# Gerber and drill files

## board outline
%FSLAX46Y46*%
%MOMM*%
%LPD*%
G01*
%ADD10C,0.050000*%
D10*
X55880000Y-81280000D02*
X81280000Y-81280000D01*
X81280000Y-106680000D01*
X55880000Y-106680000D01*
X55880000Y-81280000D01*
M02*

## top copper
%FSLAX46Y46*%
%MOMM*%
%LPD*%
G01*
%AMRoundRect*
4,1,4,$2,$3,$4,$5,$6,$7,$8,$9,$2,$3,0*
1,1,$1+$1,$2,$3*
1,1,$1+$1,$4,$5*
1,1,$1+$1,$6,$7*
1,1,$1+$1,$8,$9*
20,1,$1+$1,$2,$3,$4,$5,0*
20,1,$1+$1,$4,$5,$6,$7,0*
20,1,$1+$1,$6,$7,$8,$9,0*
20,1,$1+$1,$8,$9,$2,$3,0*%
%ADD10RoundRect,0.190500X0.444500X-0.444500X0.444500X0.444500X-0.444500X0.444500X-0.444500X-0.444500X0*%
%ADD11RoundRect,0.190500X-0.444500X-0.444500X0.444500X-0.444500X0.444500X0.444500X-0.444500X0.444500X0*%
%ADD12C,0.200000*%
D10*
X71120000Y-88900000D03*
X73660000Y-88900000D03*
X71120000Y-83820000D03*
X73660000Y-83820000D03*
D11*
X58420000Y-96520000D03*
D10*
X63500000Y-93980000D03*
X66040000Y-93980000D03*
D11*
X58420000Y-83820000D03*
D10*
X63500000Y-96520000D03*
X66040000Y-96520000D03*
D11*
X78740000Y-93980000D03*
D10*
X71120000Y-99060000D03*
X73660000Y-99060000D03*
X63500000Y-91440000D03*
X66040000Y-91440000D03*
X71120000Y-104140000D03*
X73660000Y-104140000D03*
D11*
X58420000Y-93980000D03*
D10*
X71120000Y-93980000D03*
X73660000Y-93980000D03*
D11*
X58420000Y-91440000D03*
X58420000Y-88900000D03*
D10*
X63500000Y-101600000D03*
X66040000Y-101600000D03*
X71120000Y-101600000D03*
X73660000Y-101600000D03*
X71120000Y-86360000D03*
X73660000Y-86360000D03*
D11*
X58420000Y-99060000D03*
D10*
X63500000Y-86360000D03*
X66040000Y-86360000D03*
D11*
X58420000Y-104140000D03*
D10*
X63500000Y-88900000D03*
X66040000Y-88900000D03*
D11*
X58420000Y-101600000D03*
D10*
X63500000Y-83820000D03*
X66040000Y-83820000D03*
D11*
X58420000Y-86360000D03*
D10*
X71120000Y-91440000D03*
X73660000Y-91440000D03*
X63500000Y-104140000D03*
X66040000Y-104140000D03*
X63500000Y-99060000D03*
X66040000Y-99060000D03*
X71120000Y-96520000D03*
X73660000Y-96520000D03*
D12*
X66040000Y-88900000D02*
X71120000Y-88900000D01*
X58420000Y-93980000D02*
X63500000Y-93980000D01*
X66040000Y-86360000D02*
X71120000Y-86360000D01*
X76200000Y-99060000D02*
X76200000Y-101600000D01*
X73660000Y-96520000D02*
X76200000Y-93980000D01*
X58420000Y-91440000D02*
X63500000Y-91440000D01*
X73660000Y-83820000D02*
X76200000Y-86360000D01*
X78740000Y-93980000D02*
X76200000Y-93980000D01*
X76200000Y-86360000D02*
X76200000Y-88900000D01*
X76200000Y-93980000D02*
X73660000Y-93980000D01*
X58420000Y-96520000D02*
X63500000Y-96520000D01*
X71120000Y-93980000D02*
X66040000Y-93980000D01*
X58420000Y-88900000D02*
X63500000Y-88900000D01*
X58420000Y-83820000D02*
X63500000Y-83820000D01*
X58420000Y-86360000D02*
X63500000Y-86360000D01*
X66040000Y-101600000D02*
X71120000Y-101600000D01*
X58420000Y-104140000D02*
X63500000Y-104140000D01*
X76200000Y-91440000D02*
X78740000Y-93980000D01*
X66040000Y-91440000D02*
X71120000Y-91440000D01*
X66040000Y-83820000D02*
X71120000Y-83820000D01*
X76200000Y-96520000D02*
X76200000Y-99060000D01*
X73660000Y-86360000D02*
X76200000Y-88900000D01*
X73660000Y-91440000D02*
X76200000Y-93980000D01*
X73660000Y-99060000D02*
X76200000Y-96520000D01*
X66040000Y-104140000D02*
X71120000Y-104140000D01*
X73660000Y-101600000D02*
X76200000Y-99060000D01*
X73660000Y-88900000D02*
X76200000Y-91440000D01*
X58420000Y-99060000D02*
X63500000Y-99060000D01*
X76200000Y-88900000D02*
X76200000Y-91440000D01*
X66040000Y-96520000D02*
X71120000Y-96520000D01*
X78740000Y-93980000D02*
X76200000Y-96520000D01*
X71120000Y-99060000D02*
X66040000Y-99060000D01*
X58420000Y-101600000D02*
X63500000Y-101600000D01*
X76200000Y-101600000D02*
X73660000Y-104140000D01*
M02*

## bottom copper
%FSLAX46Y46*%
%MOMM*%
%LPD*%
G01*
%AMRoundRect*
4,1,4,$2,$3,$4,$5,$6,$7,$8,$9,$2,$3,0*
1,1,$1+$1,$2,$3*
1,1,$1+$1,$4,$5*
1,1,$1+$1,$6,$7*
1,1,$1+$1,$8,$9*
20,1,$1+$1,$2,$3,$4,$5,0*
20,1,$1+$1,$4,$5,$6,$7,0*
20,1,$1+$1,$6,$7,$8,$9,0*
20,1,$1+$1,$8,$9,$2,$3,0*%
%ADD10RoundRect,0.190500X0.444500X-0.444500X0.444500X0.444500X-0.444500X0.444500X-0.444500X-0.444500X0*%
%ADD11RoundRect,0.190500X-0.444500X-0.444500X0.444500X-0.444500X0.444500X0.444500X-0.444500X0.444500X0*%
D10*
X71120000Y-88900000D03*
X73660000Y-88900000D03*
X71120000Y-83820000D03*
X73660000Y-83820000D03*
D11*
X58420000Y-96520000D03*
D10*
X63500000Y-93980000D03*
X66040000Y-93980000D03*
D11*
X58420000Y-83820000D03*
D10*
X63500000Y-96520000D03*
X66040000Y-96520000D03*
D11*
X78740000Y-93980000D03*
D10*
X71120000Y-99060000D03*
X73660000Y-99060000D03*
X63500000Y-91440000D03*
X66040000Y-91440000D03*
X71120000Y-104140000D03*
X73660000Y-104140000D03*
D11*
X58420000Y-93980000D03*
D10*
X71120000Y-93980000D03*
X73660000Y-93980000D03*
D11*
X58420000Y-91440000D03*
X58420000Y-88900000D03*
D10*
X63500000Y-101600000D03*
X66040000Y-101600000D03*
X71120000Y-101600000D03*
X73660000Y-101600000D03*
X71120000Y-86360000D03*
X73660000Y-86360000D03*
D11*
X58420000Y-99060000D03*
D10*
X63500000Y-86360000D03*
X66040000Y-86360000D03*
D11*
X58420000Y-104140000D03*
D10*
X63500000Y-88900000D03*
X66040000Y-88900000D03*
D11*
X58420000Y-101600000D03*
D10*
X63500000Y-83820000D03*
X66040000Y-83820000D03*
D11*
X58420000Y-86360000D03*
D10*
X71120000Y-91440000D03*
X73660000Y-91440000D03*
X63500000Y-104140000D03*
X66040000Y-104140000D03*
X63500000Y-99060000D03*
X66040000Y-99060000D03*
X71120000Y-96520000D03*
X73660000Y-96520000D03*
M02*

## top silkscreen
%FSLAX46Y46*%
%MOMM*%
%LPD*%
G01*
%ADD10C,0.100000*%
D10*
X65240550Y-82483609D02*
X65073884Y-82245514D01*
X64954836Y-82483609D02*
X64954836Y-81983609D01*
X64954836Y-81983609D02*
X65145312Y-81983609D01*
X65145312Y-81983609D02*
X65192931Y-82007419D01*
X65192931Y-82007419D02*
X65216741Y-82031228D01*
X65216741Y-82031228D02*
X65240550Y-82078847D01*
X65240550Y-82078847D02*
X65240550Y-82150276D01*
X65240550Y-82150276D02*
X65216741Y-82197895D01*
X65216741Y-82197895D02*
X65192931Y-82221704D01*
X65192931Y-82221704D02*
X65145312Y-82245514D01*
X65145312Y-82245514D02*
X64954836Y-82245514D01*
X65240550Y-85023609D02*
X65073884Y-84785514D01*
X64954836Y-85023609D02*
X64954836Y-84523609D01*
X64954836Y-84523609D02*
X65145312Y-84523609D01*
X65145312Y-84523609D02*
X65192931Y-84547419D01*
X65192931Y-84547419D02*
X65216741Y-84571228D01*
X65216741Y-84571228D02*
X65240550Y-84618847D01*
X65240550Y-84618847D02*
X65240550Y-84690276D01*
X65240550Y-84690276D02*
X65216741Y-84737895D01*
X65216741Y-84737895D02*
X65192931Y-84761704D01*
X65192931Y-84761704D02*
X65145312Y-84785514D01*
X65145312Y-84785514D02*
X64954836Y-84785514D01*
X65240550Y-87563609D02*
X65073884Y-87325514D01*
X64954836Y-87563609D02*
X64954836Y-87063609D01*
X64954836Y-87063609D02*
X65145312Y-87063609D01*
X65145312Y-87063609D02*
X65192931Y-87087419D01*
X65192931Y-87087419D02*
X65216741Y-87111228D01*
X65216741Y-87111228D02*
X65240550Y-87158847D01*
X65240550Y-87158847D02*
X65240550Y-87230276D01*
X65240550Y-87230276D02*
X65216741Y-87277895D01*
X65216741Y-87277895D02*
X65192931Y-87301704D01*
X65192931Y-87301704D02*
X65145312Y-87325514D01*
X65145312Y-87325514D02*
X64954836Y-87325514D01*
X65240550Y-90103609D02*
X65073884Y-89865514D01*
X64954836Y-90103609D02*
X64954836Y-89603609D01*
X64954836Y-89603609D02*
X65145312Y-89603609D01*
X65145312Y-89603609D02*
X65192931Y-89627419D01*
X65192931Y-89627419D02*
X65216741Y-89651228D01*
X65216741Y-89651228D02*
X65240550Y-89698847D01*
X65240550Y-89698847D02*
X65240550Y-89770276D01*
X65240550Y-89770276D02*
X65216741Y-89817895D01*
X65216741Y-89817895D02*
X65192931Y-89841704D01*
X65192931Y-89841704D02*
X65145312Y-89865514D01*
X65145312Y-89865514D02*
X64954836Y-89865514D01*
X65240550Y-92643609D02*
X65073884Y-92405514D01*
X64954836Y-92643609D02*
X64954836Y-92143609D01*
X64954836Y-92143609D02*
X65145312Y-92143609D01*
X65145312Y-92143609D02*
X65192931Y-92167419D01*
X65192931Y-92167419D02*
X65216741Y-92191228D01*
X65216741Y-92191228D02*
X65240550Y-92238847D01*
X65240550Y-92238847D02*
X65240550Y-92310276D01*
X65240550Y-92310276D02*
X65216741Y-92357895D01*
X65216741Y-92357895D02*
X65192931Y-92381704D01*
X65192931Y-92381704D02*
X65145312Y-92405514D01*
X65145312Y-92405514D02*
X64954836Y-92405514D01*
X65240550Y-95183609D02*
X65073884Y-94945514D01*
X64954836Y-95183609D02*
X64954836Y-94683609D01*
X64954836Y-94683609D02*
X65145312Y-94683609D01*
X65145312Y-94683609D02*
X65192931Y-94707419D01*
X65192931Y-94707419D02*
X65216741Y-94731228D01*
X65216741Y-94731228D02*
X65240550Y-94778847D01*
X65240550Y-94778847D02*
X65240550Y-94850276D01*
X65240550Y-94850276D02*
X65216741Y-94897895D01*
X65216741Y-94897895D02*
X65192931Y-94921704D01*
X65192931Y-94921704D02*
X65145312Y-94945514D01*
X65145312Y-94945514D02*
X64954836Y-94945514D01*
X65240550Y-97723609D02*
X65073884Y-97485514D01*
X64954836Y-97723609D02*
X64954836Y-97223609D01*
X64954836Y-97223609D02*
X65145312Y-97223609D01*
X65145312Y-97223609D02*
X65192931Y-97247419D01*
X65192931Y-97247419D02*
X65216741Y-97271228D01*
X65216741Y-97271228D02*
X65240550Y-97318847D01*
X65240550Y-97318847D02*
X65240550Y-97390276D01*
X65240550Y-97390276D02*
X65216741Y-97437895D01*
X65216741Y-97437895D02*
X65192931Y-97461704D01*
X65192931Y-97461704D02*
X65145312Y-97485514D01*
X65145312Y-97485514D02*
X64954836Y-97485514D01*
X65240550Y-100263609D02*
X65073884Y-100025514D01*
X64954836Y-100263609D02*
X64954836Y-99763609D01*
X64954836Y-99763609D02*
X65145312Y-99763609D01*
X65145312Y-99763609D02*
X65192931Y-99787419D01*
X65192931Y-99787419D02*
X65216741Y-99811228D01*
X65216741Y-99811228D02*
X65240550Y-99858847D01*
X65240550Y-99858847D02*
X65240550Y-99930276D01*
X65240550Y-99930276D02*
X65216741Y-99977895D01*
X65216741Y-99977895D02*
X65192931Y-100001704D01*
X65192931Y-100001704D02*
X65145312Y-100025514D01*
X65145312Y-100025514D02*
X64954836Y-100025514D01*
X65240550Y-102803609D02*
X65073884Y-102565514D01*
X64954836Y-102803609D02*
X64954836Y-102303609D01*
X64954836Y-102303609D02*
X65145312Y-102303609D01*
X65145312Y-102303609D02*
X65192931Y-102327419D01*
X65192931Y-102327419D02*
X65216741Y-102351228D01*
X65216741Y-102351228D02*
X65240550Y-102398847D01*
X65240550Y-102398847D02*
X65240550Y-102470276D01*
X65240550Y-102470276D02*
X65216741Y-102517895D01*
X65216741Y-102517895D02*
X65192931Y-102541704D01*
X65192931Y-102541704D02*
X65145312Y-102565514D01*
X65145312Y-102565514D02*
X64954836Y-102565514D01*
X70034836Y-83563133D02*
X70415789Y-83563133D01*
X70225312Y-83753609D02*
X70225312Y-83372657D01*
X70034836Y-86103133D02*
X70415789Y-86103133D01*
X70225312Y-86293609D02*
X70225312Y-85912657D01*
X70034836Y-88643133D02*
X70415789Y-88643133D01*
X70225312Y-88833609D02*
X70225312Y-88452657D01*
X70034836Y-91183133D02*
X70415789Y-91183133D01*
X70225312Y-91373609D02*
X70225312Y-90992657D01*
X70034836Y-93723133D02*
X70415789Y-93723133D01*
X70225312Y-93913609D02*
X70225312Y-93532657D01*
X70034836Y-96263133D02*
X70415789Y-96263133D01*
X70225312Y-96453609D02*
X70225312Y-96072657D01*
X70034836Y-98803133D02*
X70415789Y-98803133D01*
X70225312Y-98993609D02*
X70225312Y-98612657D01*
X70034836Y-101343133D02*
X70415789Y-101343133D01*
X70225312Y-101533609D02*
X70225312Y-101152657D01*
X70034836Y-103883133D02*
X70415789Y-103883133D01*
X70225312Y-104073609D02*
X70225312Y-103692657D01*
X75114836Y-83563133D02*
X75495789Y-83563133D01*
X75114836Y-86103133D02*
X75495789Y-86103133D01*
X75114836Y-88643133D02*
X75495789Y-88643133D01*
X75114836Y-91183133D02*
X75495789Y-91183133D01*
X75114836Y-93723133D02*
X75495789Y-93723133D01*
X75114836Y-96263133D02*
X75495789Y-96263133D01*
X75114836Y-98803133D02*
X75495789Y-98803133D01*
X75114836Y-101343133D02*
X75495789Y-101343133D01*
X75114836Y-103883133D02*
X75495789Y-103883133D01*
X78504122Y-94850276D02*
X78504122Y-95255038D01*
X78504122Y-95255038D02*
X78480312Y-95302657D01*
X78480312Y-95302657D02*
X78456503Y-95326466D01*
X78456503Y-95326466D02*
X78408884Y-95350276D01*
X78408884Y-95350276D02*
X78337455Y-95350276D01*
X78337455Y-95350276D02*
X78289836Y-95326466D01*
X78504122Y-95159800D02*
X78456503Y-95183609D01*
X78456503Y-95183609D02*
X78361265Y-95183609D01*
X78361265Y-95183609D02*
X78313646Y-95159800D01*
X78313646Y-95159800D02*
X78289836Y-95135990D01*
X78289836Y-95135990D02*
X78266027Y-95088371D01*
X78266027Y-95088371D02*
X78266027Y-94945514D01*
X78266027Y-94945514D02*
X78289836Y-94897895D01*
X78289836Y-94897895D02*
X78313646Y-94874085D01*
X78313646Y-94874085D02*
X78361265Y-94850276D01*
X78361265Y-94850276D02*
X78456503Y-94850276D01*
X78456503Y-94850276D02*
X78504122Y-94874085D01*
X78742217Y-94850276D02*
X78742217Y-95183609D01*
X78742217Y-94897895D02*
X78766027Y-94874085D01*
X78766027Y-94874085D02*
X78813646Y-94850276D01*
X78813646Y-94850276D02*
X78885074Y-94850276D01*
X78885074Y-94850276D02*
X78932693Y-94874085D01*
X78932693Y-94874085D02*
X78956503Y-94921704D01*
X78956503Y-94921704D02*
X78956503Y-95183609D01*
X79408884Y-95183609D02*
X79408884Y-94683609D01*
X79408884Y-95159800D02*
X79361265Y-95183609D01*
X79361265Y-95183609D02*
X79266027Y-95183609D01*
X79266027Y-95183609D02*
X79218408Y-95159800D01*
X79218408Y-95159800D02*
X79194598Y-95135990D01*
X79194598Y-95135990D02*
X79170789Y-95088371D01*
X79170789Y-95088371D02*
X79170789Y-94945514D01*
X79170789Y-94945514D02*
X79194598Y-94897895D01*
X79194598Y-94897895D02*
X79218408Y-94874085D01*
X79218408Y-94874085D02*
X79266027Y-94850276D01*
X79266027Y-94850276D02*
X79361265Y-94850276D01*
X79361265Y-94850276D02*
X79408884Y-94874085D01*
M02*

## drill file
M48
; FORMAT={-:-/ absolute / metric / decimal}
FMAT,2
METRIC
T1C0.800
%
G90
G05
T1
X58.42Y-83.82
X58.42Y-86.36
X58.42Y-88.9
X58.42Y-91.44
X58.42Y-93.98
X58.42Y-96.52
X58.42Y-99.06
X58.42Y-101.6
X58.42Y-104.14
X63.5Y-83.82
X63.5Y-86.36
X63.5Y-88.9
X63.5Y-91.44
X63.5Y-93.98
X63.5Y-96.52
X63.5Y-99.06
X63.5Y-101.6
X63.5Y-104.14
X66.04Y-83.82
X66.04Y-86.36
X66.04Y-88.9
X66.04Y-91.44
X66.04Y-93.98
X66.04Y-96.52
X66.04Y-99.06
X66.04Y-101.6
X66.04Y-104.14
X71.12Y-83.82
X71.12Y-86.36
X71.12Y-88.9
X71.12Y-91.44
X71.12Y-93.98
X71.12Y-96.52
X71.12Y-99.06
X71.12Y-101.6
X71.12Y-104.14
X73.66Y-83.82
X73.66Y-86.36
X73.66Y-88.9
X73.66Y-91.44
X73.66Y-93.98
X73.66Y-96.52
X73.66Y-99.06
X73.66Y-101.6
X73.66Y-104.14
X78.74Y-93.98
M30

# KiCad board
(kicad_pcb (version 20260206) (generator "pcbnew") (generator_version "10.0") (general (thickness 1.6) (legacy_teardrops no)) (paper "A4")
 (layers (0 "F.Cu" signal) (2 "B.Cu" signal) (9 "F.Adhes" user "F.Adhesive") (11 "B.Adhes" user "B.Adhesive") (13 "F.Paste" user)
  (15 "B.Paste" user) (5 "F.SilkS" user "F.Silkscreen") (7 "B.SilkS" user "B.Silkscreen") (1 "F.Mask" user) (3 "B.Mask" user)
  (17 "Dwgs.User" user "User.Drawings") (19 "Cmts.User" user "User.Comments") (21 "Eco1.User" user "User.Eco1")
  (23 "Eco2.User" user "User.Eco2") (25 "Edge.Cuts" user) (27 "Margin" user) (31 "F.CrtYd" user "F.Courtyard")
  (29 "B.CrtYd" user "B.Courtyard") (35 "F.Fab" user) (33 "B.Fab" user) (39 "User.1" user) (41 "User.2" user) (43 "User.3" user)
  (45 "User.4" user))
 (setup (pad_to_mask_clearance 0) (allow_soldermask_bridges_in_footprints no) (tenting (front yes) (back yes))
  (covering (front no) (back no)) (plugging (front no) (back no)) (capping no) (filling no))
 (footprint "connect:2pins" (layer "F.Cu") (at 68.58 88.9 90)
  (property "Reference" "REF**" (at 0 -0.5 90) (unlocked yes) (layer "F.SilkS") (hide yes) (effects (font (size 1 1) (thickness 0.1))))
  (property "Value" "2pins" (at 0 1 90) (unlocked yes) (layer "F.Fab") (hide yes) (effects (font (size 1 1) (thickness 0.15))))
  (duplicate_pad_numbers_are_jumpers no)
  (pad "1" thru_hole roundrect (at 0 2.54 90) (size 1.27 1.27) (drill 0.8) (layers "*.Cu" "*.Mask") (remove_unused_layers no)
   (roundrect_rratio 0.15))
  (pad "2" thru_hole roundrect (at 0 5.08 90) (size 1.27 1.27) (drill 0.8) (layers "*.Cu" "*.Mask") (remove_unused_layers no)
   (roundrect_rratio 0.15)))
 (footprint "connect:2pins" (layer "F.Cu") (at 68.58 83.82 90)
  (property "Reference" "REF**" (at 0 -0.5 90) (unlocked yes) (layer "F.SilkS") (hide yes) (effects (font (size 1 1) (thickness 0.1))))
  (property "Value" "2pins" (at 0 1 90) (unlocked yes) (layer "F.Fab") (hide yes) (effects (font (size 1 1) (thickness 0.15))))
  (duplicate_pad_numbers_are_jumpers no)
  (pad "1" thru_hole roundrect (at 0 2.54 90) (size 1.27 1.27) (drill 0.8) (layers "*.Cu" "*.Mask") (remove_unused_layers no)
   (roundrect_rratio 0.15))
  (pad "2" thru_hole roundrect (at 0 5.08 90) (size 1.27 1.27) (drill 0.8) (layers "*.Cu" "*.Mask") (remove_unused_layers no)
   (roundrect_rratio 0.15)))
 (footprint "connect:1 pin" (layer "F.Cu") (at 58.42 93.98)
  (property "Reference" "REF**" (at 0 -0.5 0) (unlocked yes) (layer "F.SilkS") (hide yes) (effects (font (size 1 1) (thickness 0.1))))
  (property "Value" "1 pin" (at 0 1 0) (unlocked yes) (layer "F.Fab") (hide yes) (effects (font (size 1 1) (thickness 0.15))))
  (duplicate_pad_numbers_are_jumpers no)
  (pad "1" thru_hole roundrect (at 0 2.54) (size 1.27 1.27) (drill 0.8) (layers "*.Cu" "*.Mask") (remove_unused_layers no)
   (roundrect_rratio 0.15)))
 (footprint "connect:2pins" (layer "F.Cu") (at 60.96 93.98 90)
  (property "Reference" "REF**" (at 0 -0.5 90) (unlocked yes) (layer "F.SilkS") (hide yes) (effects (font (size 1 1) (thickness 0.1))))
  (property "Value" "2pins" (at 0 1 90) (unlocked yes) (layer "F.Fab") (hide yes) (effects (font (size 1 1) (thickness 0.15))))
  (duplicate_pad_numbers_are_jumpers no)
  (pad "1" thru_hole roundrect (at 0 2.54 90) (size 1.27 1.27) (drill 0.8) (layers "*.Cu" "*.Mask") (remove_unused_layers no)
   (roundrect_rratio 0.15))
  (pad "2" thru_hole roundrect (at 0 5.08 90) (size 1.27 1.27) (drill 0.8) (layers "*.Cu" "*.Mask") (remove_unused_layers no)
   (roundrect_rratio 0.15)))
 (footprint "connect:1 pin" (layer "F.Cu") (at 58.42 81.28)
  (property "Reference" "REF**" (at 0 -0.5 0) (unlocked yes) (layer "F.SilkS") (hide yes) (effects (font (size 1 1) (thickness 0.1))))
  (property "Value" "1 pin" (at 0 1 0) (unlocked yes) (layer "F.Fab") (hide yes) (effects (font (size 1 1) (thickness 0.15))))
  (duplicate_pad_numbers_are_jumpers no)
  (pad "1" thru_hole roundrect (at 0 2.54) (size 1.27 1.27) (drill 0.8) (layers "*.Cu" "*.Mask") (remove_unused_layers no)
   (roundrect_rratio 0.15)))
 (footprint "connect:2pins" (layer "F.Cu") (at 60.96 96.52 90)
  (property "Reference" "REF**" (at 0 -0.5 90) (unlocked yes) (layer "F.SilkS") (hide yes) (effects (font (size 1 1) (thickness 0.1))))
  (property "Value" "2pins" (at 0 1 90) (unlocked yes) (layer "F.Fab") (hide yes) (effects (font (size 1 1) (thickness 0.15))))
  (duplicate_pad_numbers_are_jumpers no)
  (pad "1" thru_hole roundrect (at 0 2.54 90) (size 1.27 1.27) (drill 0.8) (layers "*.Cu" "*.Mask") (remove_unused_layers no)
   (roundrect_rratio 0.15))
  (pad "2" thru_hole roundrect (at 0 5.08 90) (size 1.27 1.27) (drill 0.8) (layers "*.Cu" "*.Mask") (remove_unused_layers no)
   (roundrect_rratio 0.15)))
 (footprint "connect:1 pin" (layer "F.Cu") (at 78.74 91.44)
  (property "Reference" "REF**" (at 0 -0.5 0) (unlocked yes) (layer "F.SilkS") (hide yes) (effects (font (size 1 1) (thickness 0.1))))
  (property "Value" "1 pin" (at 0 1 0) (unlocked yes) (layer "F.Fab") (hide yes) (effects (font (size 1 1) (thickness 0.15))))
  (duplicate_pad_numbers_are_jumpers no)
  (pad "1" thru_hole roundrect (at 0 2.54) (size 1.27 1.27) (drill 0.8) (layers "*.Cu" "*.Mask") (remove_unused_layers no)
   (roundrect_rratio 0.15)))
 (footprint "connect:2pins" (layer "F.Cu") (at 68.58 99.06 90)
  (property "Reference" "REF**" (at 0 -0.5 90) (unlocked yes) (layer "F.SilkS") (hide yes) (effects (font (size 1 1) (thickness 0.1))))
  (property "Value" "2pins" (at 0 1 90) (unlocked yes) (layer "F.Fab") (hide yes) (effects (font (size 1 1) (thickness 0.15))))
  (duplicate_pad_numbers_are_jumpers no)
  (pad "1" thru_hole roundrect (at 0 2.54 90) (size 1.27 1.27) (drill 0.8) (layers "*.Cu" "*.Mask") (remove_unused_layers no)
   (roundrect_rratio 0.15))
  (pad "2" thru_hole roundrect (at 0 5.08 90) (size 1.27 1.27) (drill 0.8) (layers "*.Cu" "*.Mask") (remove_unused_layers no)
   (roundrect_rratio 0.15)))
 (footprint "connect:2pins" (layer "F.Cu") (at 60.96 91.44 90)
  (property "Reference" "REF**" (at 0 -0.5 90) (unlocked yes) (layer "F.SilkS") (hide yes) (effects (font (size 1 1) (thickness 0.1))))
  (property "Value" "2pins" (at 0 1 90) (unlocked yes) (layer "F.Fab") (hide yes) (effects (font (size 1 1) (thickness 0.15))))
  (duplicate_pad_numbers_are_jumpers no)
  (pad "1" thru_hole roundrect (at 0 2.54 90) (size 1.27 1.27) (drill 0.8) (layers "*.Cu" "*.Mask") (remove_unused_layers no)
   (roundrect_rratio 0.15))
  (pad "2" thru_hole roundrect (at 0 5.08 90) (size 1.27 1.27) (drill 0.8) (layers "*.Cu" "*.Mask") (remove_unused_layers no)
   (roundrect_rratio 0.15)))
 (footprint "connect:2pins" (layer "F.Cu") (at 68.58 104.14 90)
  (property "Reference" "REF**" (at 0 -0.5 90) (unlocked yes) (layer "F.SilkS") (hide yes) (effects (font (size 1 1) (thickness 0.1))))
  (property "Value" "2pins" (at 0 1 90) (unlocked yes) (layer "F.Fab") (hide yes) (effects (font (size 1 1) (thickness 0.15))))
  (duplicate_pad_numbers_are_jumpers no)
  (pad "1" thru_hole roundrect (at 0 2.54 90) (size 1.27 1.27) (drill 0.8) (layers "*.Cu" "*.Mask") (remove_unused_layers no)
   (roundrect_rratio 0.15))
  (pad "2" thru_hole roundrect (at 0 5.08 90) (size 1.27 1.27) (drill 0.8) (layers "*.Cu" "*.Mask") (remove_unused_layers no)
   (roundrect_rratio 0.15)))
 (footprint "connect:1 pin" (layer "F.Cu") (at 58.42 91.44)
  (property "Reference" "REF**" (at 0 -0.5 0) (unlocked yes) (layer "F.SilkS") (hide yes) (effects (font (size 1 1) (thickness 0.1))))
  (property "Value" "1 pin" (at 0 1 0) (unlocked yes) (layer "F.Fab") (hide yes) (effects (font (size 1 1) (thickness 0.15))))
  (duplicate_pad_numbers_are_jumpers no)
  (pad "1" thru_hole roundrect (at 0 2.54) (size 1.27 1.27) (drill 0.8) (layers "*.Cu" "*.Mask") (remove_unused_layers no)
   (roundrect_rratio 0.15)))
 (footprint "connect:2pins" (layer "F.Cu") (at 68.58 93.98 90)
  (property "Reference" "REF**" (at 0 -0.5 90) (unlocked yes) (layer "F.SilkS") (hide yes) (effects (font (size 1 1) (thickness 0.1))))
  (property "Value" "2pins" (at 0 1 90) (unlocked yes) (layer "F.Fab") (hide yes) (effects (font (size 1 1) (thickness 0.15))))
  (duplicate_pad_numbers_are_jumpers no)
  (pad "1" thru_hole roundrect (at 0 2.54 90) (size 1.27 1.27) (drill 0.8) (layers "*.Cu" "*.Mask") (remove_unused_layers no)
   (roundrect_rratio 0.15))
  (pad "2" thru_hole roundrect (at 0 5.08 90) (size 1.27 1.27) (drill 0.8) (layers "*.Cu" "*.Mask") (remove_unused_layers no)
   (roundrect_rratio 0.15)))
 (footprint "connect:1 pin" (layer "F.Cu") (at 58.42 88.9)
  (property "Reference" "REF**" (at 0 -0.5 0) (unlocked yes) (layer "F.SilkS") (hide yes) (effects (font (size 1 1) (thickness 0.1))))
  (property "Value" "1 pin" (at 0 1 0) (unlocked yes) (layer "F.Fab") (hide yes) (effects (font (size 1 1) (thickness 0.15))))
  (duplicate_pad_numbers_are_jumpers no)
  (pad "1" thru_hole roundrect (at 0 2.54) (size 1.27 1.27) (drill 0.8) (layers "*.Cu" "*.Mask") (remove_unused_layers no)
   (roundrect_rratio 0.15)))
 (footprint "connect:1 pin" (layer "F.Cu") (at 58.42 86.36)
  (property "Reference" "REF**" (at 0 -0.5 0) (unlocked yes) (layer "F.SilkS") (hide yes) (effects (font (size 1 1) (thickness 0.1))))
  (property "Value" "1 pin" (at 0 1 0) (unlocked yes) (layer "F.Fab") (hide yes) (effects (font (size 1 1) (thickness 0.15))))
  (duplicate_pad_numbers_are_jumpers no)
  (pad "1" thru_hole roundrect (at 0 2.54) (size 1.27 1.27) (drill 0.8) (layers "*.Cu" "*.Mask") (remove_unused_layers no)
   (roundrect_rratio 0.15)))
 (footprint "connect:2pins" (layer "F.Cu") (at 60.96 101.6 90)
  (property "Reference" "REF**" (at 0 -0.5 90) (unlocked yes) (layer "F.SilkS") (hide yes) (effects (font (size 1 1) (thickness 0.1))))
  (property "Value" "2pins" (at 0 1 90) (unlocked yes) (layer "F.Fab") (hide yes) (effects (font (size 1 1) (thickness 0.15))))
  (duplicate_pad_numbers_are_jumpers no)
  (pad "1" thru_hole roundrect (at 0 2.54 90) (size 1.27 1.27) (drill 0.8) (layers "*.Cu" "*.Mask") (remove_unused_layers no)
   (roundrect_rratio 0.15))
  (pad "2" thru_hole roundrect (at 0 5.08 90) (size 1.27 1.27) (drill 0.8) (layers "*.Cu" "*.Mask") (remove_unused_layers no)
   (roundrect_rratio 0.15)))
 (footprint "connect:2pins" (layer "F.Cu") (at 68.58 101.6 90)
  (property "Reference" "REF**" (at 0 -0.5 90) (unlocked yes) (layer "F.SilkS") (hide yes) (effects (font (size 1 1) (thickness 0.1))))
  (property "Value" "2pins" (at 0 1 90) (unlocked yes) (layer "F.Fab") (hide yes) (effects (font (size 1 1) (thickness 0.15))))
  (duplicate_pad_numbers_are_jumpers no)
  (pad "1" thru_hole roundrect (at 0 2.54 90) (size 1.27 1.27) (drill 0.8) (layers "*.Cu" "*.Mask") (remove_unused_layers no)
   (roundrect_rratio 0.15))
  (pad "2" thru_hole roundrect (at 0 5.08 90) (size 1.27 1.27) (drill 0.8) (layers "*.Cu" "*.Mask") (remove_unused_layers no)
   (roundrect_rratio 0.15)))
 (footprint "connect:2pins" (layer "F.Cu") (at 68.58 86.36 90)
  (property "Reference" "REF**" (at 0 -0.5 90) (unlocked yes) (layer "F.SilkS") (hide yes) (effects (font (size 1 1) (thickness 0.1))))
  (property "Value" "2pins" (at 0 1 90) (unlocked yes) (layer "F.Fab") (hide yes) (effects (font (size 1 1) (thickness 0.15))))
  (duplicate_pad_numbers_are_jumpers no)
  (pad "1" thru_hole roundrect (at 0 2.54 90) (size 1.27 1.27) (drill 0.8) (layers "*.Cu" "*.Mask") (remove_unused_layers no)
   (roundrect_rratio 0.15))
  (pad "2" thru_hole roundrect (at 0 5.08 90) (size 1.27 1.27) (drill 0.8) (layers "*.Cu" "*.Mask") (remove_unused_layers no)
   (roundrect_rratio 0.15)))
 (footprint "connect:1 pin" (layer "F.Cu") (at 58.42 96.52)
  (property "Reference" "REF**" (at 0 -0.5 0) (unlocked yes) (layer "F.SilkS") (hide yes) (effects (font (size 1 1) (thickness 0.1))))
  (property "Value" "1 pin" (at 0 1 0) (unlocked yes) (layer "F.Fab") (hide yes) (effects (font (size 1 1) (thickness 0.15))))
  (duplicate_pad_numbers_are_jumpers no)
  (pad "1" thru_hole roundrect (at 0 2.54) (size 1.27 1.27) (drill 0.8) (layers "*.Cu" "*.Mask") (remove_unused_layers no)
   (roundrect_rratio 0.15)))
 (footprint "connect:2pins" (layer "F.Cu") (at 60.96 86.36 90)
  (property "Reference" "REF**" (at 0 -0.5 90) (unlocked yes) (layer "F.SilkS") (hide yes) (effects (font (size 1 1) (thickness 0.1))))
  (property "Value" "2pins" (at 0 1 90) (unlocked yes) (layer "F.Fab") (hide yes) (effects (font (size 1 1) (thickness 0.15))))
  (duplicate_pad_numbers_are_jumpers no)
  (pad "1" thru_hole roundrect (at 0 2.54 90) (size 1.27 1.27) (drill 0.8) (layers "*.Cu" "*.Mask") (remove_unused_layers no)
   (roundrect_rratio 0.15))
  (pad "2" thru_hole roundrect (at 0 5.08 90) (size 1.27 1.27) (drill 0.8) (layers "*.Cu" "*.Mask") (remove_unused_layers no)
   (roundrect_rratio 0.15)))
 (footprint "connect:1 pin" (layer "F.Cu") (at 58.42 101.6)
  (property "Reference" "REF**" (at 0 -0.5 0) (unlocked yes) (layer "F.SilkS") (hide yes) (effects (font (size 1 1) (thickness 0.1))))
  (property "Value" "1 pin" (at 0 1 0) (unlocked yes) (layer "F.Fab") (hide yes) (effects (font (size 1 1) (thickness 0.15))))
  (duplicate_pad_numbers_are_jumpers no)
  (pad "1" thru_hole roundrect (at 0 2.54) (size 1.27 1.27) (drill 0.8) (layers "*.Cu" "*.Mask") (remove_unused_layers no)
   (roundrect_rratio 0.15)))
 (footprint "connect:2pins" (layer "F.Cu") (at 60.96 88.9 90)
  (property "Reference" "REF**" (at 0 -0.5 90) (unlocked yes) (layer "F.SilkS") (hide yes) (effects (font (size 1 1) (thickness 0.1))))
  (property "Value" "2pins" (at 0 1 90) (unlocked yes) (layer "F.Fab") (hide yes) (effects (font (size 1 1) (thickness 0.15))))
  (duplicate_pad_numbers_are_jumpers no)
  (pad "1" thru_hole roundrect (at 0 2.54 90) (size 1.27 1.27) (drill 0.8) (layers "*.Cu" "*.Mask") (remove_unused_layers no)
   (roundrect_rratio 0.15))
  (pad "2" thru_hole roundrect (at 0 5.08 90) (size 1.27 1.27) (drill 0.8) (layers "*.Cu" "*.Mask") (remove_unused_layers no)
   (roundrect_rratio 0.15)))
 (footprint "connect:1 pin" (layer "F.Cu") (at 58.42 99.06)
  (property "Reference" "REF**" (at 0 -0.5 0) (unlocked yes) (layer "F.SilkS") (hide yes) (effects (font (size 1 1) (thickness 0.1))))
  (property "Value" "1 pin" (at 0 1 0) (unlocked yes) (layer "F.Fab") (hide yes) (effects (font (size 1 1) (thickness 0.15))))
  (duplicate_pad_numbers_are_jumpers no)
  (pad "1" thru_hole roundrect (at 0 2.54) (size 1.27 1.27) (drill 0.8) (layers "*.Cu" "*.Mask") (remove_unused_layers no)
   (roundrect_rratio 0.15)))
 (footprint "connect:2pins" (layer "F.Cu") (at 60.96 83.82 90)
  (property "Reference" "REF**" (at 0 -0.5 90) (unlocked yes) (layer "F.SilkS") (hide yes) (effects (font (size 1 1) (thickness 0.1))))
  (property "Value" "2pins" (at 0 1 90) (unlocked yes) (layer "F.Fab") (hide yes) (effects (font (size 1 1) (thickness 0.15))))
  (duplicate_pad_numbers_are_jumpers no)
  (pad "1" thru_hole roundrect (at 0 2.54 90) (size 1.27 1.27) (drill 0.8) (layers "*.Cu" "*.Mask") (remove_unused_layers no)
   (roundrect_rratio 0.15))
  (pad "2" thru_hole roundrect (at 0 5.08 90) (size 1.27 1.27) (drill 0.8) (layers "*.Cu" "*.Mask") (remove_unused_layers no)
   (roundrect_rratio 0.15)))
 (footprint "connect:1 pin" (layer "F.Cu") (at 58.42 83.82)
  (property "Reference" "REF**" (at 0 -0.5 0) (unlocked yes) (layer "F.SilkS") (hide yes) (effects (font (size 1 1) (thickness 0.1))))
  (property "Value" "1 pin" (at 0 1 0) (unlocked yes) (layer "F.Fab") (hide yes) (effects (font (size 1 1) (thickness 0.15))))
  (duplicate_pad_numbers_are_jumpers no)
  (pad "1" thru_hole roundrect (at 0 2.54) (size 1.27 1.27) (drill 0.8) (layers "*.Cu" "*.Mask") (remove_unused_layers no)
   (roundrect_rratio 0.15)))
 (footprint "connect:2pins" (layer "F.Cu") (at 68.58 91.44 90)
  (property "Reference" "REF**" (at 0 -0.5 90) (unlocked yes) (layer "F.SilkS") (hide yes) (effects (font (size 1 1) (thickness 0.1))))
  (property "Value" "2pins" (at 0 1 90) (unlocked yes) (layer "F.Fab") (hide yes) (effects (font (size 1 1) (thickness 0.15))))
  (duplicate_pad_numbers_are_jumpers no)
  (pad "1" thru_hole roundrect (at 0 2.54 90) (size 1.27 1.27) (drill 0.8) (layers "*.Cu" "*.Mask") (remove_unused_layers no)
   (roundrect_rratio 0.15))
  (pad "2" thru_hole roundrect (at 0 5.08 90) (size 1.27 1.27) (drill 0.8) (layers "*.Cu" "*.Mask") (remove_unused_layers no)
   (roundrect_rratio 0.15)))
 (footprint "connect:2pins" (layer "F.Cu") (at 60.96 104.14 90)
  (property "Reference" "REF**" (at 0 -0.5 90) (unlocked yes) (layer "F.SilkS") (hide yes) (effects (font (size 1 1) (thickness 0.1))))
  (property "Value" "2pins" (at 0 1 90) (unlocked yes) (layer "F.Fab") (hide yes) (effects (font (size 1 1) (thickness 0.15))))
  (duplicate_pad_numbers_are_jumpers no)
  (pad "1" thru_hole roundrect (at 0 2.54 90) (size 1.27 1.27) (drill 0.8) (layers "*.Cu" "*.Mask") (remove_unused_layers no)
   (roundrect_rratio 0.15))
  (pad "2" thru_hole roundrect (at 0 5.08 90) (size 1.27 1.27) (drill 0.8) (layers "*.Cu" "*.Mask") (remove_unused_layers no)
   (roundrect_rratio 0.15)))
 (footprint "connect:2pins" (layer "F.Cu") (at 60.96 99.06 90)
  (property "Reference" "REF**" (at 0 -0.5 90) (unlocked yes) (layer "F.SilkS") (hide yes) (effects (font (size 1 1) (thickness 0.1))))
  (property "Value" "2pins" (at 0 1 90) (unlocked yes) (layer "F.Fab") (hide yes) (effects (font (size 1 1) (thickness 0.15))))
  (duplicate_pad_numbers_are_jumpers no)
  (pad "1" thru_hole roundrect (at 0 2.54 90) (size 1.27 1.27) (drill 0.8) (layers "*.Cu" "*.Mask") (remove_unused_layers no)
   (roundrect_rratio 0.15))
  (pad "2" thru_hole roundrect (at 0 5.08 90) (size 1.27 1.27) (drill 0.8) (layers "*.Cu" "*.Mask") (remove_unused_layers no)
   (roundrect_rratio 0.15)))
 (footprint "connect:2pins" (layer "F.Cu") (at 68.58 96.52 90)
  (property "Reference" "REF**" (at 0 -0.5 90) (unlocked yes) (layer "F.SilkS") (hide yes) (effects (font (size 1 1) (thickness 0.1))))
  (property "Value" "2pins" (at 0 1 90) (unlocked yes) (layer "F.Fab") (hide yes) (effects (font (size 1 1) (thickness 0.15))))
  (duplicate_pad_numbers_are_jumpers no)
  (pad "1" thru_hole roundrect (at 0 2.54 90) (size 1.27 1.27) (drill 0.8) (layers "*.Cu" "*.Mask") (remove_unused_layers no)
   (roundrect_rratio 0.15))
  (pad "2" thru_hole roundrect (at 0 5.08 90) (size 1.27 1.27) (drill 0.8) (layers "*.Cu" "*.Mask") (remove_unused_layers no)
   (roundrect_rratio 0.15)))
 (gr_rect (start 55.88 81.28) (end 81.28 106.68) (stroke (width 0.05) (type default)) (fill no) (layer "Edge.Cuts"))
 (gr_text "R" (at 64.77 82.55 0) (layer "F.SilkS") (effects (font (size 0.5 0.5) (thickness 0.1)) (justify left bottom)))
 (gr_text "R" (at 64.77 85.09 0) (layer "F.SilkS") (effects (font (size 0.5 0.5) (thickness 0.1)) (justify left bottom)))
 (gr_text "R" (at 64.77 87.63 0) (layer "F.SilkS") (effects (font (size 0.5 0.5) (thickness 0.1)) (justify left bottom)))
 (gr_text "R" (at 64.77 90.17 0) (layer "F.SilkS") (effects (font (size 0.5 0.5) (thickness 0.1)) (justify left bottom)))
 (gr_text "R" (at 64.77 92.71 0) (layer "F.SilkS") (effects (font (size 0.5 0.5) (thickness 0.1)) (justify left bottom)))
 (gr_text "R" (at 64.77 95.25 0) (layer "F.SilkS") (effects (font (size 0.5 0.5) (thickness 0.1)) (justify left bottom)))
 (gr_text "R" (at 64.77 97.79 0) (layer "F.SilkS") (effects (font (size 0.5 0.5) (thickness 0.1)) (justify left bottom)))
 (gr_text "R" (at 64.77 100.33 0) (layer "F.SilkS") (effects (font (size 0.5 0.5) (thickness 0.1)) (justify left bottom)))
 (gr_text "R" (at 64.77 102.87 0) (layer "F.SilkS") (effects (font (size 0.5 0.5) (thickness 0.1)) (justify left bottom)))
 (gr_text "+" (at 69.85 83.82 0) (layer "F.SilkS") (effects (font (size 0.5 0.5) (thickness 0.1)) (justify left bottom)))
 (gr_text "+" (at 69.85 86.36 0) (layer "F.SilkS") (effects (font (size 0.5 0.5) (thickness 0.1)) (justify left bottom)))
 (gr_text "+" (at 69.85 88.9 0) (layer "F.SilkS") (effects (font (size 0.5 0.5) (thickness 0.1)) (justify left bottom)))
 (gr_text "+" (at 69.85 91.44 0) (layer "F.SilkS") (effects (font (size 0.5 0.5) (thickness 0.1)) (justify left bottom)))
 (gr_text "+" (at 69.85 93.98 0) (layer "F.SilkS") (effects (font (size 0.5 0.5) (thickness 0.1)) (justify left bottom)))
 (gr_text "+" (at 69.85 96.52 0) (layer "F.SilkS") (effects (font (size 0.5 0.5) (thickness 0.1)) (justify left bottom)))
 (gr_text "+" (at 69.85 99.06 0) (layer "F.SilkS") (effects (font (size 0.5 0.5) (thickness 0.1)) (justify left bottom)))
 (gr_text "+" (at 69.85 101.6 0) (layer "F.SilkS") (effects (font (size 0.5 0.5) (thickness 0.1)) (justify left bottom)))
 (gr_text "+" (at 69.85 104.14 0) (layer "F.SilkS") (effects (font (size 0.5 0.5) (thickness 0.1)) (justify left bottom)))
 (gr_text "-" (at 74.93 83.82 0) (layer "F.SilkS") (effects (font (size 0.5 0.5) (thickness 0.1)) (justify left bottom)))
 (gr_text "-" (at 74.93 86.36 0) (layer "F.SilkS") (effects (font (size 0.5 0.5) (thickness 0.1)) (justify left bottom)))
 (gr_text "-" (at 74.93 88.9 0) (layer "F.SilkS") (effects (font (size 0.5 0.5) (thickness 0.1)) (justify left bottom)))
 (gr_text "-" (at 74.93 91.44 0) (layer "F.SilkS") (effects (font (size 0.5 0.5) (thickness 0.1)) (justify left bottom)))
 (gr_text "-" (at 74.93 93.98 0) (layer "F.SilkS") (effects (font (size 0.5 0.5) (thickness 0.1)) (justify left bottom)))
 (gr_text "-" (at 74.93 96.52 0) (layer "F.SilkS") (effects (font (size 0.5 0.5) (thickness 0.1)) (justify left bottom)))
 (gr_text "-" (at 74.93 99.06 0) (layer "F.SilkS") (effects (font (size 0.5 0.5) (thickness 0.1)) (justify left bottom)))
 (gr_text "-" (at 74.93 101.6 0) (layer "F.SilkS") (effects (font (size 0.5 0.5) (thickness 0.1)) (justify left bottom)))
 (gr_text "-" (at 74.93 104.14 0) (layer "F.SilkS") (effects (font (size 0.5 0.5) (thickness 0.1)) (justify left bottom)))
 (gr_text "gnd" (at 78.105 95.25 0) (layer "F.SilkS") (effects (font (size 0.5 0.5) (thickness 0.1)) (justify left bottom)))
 (segment (start 66.04 88.9) (end 71.12 88.9) (width 0.2) (layer "F.Cu") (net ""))
 (segment (start 58.42 93.98) (end 63.5 93.98) (width 0.2) (layer "F.Cu") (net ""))
 (segment (start 66.04 86.36) (end 71.12 86.36) (width 0.2) (layer "F.Cu") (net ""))
 (segment (start 76.2 99.06) (end 76.2 101.6) (width 0.2) (layer "F.Cu") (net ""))
 (segment (start 73.66 96.52) (end 76.2 93.98) (width 0.2) (layer "F.Cu") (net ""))
 (segment (start 58.42 91.44) (end 63.5 91.44) (width 0.2) (layer "F.Cu") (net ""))
 (segment (start 73.66 83.82) (end 76.2 86.36) (width 0.2) (layer "F.Cu") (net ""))
 (segment (start 78.74 93.98) (end 76.2 93.98) (width 0.2) (layer "F.Cu") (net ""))
 (segment (start 76.2 86.36) (end 76.2 88.9) (width 0.2) (layer "F.Cu") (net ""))
 (segment (start 76.2 93.98) (end 73.66 93.98) (width 0.2) (layer "F.Cu") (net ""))
 (segment (start 58.42 96.52) (end 63.5 96.52) (width 0.2) (layer "F.Cu") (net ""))
 (segment (start 71.12 93.98) (end 66.04 93.98) (width 0.2) (layer "F.Cu") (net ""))
 (segment (start 58.42 88.9) (end 63.5 88.9) (width 0.2) (layer "F.Cu") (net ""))
 (segment (start 58.42 83.82) (end 63.5 83.82) (width 0.2) (layer "F.Cu") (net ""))
 (segment (start 58.42 86.36) (end 63.5 86.36) (width 0.2) (layer "F.Cu") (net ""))
 (segment (start 66.04 101.6) (end 71.12 101.6) (width 0.2) (layer "F.Cu") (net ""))
 (segment (start 58.42 104.14) (end 63.5 104.14) (width 0.2) (layer "F.Cu") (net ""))
 (segment (start 76.2 91.44) (end 78.74 93.98) (width 0.2) (layer "F.Cu") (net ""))
 (segment (start 66.04 91.44) (end 71.12 91.44) (width 0.2) (layer "F.Cu") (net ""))
 (segment (start 66.04 83.82) (end 71.12 83.82) (width 0.2) (layer "F.Cu") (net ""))
 (segment (start 76.2 96.52) (end 76.2 99.06) (width 0.2) (layer "F.Cu") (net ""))
 (segment (start 73.66 86.36) (end 76.2 88.9) (width 0.2) (layer "F.Cu") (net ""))
 (segment (start 73.66 91.44) (end 76.2 93.98) (width 0.2) (layer "F.Cu") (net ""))
 (segment (start 73.66 99.06) (end 76.2 96.52) (width 0.2) (layer "F.Cu") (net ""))
 (segment (start 66.04 104.14) (end 71.12 104.14) (width 0.2) (layer "F.Cu") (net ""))
 (segment (start 73.66 101.6) (end 76.2 99.06) (width 0.2) (layer "F.Cu") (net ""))
 (segment (start 73.66 88.9) (end 76.2 91.44) (width 0.2) (layer "F.Cu") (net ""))
 (segment (start 58.42 99.06) (end 63.5 99.06) (width 0.2) (layer "F.Cu") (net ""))
 (segment (start 76.2 88.9) (end 76.2 91.44) (width 0.2) (layer "F.Cu") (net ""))
 (segment (start 66.04 96.52) (end 71.12 96.52) (width 0.2) (layer "F.Cu") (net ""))
 (segment (start 78.74 93.98) (end 76.2 96.52) (width 0.2) (layer "F.Cu") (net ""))
 (segment (start 71.12 99.06) (end 66.04 99.06) (width 0.2) (layer "F.Cu") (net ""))
 (segment (start 58.42 101.6) (end 63.5 101.6) (width 0.2) (layer "F.Cu") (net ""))
 (segment (start 76.2 101.6) (end 73.66 104.14) (width 0.2) (layer "F.Cu") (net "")))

